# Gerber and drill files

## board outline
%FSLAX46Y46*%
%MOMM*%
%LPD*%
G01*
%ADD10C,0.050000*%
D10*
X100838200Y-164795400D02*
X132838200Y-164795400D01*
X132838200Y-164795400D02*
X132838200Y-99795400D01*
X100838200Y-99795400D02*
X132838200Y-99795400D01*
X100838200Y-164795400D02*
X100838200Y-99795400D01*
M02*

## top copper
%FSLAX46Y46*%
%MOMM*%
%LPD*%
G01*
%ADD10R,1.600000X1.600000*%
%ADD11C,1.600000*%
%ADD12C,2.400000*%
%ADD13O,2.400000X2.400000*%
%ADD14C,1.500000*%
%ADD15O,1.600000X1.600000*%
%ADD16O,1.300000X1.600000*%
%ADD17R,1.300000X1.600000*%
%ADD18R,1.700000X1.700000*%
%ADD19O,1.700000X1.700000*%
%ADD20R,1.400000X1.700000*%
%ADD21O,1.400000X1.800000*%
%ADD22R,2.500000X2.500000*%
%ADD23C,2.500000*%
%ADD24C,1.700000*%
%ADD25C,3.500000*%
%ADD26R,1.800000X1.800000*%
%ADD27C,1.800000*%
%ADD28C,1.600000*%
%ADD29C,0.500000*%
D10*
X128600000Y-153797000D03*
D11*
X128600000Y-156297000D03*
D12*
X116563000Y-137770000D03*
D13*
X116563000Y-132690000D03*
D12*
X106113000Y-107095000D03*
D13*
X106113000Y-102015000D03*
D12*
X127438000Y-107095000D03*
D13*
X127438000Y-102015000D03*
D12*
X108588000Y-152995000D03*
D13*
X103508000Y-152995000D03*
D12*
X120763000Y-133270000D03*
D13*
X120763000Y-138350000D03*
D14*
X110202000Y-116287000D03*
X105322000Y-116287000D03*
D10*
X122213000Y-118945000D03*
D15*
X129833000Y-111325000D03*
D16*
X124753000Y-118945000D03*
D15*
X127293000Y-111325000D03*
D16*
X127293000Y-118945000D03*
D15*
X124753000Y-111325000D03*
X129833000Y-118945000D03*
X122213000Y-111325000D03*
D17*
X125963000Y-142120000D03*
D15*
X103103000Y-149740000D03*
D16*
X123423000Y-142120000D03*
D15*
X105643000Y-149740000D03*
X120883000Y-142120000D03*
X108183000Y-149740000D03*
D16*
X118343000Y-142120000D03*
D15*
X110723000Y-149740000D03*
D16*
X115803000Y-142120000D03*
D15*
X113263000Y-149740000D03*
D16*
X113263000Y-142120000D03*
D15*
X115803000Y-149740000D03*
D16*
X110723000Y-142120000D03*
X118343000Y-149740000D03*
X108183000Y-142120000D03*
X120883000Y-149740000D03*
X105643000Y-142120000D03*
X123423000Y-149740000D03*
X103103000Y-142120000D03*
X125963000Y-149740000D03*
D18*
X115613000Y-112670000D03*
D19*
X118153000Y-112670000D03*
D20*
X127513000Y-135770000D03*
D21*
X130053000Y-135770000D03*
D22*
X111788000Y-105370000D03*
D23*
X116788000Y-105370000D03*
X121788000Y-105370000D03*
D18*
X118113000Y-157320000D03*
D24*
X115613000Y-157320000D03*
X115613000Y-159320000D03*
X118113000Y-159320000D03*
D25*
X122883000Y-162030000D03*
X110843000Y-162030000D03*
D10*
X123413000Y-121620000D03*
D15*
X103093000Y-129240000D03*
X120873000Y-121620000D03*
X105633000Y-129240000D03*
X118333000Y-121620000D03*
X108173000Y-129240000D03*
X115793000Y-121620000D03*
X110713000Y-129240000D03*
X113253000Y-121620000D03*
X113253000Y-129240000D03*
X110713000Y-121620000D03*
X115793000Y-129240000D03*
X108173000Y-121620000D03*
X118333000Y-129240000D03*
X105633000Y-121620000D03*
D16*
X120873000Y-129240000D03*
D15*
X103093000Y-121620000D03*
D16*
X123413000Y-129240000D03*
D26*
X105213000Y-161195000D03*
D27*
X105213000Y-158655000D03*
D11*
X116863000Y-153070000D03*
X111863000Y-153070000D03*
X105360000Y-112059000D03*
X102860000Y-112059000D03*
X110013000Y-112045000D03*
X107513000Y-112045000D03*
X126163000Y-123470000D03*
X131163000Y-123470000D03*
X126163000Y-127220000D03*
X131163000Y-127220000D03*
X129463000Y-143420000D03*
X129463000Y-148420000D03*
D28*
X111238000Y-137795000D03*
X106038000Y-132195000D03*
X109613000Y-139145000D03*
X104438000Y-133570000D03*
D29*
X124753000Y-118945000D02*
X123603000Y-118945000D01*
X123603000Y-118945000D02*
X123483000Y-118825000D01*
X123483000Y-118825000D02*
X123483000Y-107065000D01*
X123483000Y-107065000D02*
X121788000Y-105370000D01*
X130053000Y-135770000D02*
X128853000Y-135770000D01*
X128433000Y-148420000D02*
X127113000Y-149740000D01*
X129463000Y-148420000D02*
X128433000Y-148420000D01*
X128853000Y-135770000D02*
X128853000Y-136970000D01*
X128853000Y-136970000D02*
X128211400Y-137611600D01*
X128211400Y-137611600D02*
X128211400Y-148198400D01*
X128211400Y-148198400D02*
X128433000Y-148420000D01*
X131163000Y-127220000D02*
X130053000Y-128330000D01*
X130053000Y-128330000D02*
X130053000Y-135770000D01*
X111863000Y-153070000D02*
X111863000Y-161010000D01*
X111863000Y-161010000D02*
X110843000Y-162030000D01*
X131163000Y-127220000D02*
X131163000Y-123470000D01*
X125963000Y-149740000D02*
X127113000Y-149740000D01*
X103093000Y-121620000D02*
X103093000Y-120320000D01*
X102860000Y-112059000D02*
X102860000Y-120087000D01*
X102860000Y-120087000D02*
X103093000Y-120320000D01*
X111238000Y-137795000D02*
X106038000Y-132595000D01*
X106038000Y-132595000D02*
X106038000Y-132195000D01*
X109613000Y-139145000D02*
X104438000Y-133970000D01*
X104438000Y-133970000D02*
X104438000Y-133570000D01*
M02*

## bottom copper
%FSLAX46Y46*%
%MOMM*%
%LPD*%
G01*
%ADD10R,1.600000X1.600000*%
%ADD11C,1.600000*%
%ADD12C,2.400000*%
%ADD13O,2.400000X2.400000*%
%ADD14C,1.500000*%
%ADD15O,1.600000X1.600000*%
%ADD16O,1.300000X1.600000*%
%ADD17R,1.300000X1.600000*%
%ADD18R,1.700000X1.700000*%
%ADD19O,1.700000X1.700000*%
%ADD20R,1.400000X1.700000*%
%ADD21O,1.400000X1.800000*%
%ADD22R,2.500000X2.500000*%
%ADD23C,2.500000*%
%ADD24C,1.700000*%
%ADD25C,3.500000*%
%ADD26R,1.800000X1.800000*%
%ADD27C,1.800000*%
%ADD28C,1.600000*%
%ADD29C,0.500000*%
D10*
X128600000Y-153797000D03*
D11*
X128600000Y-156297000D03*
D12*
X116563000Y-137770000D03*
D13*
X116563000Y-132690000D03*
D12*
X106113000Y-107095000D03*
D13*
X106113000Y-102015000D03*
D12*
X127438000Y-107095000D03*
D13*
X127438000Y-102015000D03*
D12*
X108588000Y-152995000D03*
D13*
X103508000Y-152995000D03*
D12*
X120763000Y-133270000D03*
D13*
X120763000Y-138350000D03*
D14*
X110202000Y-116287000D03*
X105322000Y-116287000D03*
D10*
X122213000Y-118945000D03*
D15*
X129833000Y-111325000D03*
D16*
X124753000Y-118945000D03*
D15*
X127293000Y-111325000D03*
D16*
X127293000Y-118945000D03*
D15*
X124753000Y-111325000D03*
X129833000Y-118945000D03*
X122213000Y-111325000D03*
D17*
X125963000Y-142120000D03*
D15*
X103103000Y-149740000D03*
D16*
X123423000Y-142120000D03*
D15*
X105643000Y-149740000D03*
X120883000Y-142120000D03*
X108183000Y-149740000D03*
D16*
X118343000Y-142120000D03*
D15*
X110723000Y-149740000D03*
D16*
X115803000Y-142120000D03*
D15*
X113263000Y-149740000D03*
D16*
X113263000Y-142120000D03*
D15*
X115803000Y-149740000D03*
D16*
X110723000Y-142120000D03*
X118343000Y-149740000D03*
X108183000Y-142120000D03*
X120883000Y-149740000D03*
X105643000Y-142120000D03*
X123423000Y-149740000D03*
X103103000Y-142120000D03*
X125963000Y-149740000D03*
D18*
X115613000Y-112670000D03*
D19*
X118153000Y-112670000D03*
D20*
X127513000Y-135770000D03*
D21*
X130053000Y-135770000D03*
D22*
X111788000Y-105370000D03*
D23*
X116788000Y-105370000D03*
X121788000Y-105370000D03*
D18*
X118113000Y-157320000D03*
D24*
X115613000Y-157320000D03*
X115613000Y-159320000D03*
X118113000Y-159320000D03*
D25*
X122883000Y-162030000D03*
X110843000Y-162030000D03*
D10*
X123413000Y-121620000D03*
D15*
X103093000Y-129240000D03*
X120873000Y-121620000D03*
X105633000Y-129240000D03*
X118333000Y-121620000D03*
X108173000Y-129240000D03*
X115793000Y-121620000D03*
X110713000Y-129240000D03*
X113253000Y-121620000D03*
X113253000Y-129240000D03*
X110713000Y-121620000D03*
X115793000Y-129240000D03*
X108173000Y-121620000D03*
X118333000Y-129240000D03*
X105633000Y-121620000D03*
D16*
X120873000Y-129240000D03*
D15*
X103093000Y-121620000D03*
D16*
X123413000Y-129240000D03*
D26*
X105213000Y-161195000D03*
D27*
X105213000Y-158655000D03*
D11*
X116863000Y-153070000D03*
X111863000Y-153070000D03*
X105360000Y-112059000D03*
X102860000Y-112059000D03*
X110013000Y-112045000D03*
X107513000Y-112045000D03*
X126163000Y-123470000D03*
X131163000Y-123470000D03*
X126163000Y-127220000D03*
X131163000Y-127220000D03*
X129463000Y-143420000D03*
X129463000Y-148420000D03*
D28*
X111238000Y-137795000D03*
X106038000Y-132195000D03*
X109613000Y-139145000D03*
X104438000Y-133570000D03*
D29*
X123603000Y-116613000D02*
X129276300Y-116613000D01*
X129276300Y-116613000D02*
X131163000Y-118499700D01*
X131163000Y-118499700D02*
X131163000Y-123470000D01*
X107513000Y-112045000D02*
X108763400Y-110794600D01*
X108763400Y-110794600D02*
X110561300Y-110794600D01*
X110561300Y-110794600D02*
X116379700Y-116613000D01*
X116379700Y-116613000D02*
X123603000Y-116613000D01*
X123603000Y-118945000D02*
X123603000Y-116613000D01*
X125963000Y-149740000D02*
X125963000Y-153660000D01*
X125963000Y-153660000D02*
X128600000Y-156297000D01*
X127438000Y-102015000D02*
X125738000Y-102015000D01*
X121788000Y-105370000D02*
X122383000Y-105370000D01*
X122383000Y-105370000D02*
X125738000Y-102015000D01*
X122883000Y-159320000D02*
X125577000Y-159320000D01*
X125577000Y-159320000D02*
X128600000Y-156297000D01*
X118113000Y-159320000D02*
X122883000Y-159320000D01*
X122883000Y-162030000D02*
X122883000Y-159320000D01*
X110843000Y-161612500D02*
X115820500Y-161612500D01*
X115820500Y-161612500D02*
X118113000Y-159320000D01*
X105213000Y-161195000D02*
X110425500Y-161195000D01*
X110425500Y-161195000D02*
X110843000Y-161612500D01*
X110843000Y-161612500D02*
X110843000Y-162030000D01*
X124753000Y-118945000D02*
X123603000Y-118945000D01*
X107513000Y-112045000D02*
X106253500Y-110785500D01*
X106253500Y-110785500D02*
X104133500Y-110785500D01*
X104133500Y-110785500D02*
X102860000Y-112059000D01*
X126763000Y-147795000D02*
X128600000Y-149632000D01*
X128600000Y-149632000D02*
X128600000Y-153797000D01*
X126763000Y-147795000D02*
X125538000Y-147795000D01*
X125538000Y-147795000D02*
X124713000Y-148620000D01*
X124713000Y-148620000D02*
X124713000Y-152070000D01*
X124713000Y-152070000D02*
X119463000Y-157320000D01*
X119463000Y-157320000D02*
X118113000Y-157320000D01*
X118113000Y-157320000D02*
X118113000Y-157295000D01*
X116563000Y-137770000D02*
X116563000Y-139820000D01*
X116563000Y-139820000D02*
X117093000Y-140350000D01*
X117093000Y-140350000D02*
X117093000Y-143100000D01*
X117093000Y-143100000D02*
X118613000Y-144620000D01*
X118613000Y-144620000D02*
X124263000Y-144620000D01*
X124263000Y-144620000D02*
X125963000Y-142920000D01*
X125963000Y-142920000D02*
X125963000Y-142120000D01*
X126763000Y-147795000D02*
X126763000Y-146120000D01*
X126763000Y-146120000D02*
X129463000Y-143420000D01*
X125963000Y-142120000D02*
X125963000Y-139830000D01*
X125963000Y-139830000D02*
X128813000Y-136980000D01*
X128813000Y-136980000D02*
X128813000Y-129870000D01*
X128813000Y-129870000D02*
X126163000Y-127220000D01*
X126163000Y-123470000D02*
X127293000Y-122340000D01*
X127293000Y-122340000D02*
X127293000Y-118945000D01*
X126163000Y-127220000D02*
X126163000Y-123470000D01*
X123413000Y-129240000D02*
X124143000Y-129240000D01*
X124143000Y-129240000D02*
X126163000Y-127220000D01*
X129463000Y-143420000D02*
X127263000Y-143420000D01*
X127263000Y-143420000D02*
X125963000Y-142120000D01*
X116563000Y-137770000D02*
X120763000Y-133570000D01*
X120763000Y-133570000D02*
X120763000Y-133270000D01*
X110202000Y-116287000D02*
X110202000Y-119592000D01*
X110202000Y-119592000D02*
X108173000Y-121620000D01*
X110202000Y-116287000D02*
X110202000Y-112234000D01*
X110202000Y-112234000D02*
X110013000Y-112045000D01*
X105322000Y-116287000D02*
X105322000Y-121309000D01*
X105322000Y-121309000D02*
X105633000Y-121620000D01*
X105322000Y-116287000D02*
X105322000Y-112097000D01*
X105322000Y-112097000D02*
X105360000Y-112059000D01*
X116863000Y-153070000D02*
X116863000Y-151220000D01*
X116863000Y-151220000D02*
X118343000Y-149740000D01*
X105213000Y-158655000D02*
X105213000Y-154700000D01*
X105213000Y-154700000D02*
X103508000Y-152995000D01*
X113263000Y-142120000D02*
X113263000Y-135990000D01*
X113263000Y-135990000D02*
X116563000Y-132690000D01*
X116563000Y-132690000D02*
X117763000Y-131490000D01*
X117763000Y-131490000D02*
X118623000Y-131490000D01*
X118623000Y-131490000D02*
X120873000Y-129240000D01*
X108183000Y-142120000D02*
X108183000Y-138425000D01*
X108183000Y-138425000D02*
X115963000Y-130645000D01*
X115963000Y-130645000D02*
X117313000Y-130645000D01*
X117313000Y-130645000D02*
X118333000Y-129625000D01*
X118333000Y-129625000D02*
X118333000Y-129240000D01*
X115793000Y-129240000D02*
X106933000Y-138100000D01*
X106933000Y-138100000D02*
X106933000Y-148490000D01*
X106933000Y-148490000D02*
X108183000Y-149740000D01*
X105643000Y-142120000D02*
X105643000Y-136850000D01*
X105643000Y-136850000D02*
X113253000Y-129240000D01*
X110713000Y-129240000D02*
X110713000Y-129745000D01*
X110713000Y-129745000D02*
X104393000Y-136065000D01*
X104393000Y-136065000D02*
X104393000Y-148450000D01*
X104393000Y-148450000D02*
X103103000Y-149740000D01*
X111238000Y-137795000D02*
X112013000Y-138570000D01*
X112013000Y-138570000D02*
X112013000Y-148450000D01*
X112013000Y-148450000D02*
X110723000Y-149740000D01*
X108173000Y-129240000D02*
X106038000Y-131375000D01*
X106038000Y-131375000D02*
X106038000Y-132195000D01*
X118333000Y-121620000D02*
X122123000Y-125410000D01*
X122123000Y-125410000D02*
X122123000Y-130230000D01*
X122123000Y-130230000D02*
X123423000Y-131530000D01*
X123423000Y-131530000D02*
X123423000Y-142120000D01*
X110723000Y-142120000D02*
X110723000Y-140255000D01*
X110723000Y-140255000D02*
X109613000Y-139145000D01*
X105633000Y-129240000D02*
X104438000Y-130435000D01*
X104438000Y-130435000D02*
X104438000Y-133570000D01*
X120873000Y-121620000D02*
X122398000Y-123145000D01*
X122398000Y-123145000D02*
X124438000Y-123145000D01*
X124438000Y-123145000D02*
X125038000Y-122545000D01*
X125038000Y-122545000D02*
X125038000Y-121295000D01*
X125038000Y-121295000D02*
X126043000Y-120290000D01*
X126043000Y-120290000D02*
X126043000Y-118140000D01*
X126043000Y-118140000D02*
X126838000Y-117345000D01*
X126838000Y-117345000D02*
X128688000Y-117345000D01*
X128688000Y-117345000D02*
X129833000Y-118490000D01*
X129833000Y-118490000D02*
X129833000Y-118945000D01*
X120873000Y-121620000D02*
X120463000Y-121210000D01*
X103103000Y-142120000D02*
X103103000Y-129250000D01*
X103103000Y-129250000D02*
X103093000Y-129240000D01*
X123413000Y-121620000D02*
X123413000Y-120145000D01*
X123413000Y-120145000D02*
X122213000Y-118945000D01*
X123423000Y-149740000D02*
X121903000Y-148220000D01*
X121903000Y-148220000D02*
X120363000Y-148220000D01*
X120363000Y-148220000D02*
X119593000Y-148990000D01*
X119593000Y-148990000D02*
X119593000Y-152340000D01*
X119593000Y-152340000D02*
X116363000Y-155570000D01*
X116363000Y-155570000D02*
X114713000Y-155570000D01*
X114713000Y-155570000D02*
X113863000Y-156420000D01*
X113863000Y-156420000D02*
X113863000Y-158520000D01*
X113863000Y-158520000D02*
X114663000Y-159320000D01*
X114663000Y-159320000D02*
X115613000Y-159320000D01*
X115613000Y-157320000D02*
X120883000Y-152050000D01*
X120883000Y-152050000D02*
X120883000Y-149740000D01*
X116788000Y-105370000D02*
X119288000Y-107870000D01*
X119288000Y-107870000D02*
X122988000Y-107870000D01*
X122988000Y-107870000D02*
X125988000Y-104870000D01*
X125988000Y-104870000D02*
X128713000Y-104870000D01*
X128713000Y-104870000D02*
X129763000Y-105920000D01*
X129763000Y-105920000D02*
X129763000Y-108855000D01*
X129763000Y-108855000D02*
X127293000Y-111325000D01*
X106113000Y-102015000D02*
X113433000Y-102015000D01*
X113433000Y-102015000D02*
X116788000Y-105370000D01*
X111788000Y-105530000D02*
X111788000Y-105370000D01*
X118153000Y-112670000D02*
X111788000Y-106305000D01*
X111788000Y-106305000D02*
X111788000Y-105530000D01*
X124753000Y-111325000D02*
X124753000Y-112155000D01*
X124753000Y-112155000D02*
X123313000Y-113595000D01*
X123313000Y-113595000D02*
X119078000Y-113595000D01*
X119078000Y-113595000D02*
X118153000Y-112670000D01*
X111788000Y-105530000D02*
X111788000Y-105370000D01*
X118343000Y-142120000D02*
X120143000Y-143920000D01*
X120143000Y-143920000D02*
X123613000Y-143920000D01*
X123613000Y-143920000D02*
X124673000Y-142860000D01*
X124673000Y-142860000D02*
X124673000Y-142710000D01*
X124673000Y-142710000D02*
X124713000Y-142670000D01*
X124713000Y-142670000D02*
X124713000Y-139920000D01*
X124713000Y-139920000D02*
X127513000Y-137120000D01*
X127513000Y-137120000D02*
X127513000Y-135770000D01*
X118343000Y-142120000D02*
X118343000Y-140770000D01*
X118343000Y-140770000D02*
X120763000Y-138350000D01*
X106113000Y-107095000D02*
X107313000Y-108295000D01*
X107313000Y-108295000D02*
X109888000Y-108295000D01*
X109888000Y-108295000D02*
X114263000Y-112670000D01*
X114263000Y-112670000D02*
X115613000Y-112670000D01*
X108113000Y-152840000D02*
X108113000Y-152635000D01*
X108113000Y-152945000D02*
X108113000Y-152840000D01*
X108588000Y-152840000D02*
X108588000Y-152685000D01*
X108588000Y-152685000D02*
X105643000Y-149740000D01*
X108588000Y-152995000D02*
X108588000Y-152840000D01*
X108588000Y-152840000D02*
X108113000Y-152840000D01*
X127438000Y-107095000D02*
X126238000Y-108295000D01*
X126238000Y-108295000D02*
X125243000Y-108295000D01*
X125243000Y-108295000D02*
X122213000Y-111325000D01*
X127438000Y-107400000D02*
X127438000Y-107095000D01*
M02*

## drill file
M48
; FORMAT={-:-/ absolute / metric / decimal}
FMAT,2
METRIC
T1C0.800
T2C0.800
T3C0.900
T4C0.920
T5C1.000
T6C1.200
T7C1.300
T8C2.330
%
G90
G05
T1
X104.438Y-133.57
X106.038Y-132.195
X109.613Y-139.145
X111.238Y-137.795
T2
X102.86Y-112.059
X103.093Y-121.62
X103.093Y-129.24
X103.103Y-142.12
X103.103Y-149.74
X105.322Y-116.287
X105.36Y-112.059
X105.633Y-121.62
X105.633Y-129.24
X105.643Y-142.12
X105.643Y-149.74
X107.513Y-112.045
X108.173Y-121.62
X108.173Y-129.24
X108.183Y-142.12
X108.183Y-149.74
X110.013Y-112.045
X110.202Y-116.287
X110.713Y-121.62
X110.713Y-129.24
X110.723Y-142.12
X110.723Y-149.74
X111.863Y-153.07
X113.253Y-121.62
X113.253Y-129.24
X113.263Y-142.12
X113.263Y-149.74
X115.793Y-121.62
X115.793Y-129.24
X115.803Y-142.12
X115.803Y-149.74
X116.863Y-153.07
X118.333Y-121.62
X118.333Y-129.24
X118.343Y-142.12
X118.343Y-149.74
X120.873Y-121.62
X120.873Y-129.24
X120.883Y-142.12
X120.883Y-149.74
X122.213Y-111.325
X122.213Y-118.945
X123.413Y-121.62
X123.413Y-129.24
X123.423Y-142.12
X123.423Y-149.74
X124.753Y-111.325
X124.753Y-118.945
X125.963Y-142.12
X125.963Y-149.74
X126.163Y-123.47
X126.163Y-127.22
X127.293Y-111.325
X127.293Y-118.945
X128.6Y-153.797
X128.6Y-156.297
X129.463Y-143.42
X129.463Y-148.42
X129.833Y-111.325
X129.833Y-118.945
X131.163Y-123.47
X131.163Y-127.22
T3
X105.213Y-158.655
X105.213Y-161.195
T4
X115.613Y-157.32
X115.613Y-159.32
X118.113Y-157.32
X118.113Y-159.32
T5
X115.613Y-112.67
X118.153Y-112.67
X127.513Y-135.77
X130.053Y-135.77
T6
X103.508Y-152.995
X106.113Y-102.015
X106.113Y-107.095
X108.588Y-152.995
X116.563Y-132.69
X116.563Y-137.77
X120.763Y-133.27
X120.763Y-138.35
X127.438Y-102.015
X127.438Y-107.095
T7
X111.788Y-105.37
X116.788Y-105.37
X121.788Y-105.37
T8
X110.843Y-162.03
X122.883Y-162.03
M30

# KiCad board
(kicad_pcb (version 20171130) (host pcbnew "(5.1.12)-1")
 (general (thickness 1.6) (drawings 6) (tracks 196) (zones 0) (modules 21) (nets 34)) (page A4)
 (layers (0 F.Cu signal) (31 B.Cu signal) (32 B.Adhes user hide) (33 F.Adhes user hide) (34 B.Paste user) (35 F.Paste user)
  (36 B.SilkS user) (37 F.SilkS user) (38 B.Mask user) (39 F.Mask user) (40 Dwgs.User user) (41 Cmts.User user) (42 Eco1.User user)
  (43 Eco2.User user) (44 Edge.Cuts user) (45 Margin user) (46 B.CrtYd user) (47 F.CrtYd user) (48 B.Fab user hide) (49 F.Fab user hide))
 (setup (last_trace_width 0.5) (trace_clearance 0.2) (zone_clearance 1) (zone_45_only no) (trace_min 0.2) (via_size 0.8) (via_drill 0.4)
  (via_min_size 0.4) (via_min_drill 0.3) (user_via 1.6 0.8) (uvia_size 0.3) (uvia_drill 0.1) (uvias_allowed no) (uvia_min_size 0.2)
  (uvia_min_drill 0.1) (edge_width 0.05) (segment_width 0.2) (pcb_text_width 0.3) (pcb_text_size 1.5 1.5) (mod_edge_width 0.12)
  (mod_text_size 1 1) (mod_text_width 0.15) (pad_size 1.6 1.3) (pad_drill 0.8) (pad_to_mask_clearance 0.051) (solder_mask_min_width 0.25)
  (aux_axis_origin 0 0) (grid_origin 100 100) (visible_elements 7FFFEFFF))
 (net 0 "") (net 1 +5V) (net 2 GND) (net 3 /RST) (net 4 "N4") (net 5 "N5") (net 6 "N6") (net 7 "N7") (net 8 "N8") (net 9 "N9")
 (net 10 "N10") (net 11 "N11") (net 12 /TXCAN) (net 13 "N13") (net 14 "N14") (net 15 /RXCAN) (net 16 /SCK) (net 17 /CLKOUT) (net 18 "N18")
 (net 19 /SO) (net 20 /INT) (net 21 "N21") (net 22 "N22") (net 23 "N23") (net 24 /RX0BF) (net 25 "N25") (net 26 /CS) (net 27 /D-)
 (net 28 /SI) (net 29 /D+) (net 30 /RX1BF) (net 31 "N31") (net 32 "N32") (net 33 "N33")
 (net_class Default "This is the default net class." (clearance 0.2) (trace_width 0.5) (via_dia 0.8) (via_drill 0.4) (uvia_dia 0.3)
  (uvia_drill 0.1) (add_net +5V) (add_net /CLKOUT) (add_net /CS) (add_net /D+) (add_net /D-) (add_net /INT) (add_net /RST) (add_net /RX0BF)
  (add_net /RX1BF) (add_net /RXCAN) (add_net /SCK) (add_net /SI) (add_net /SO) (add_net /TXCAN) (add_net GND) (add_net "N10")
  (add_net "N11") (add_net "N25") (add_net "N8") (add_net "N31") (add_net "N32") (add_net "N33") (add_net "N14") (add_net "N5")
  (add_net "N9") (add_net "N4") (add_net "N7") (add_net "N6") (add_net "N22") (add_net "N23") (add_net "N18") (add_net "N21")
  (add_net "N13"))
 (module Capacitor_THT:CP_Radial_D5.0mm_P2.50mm (layer F.Cu) (at 128.6 153.797 270)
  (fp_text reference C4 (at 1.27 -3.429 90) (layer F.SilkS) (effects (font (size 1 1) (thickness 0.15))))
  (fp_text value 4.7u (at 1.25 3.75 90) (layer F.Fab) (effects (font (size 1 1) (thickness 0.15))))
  (pad 1 thru_hole rect (at 0 0 270) (size 1.6 1.6) (drill 0.8) (layers *.Cu *.Mask) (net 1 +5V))
  (pad 2 thru_hole circle (at 2.5 0 270) (size 1.6 1.6) (drill 0.8) (layers *.Cu *.Mask) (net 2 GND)))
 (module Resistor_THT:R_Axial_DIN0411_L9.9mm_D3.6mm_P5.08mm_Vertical (layer F.Cu) (at 116.563 137.77 90)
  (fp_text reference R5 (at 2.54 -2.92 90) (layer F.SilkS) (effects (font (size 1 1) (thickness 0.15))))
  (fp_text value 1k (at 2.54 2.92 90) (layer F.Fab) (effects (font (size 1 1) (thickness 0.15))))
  (pad 1 thru_hole circle (at 0 0 90) (size 2.4 2.4) (drill 1.2) (layers *.Cu *.Mask) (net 1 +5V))
  (pad 2 thru_hole oval (at 5.08 0 90) (size 2.4 2.4) (drill 1.2) (layers *.Cu *.Mask) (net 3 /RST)))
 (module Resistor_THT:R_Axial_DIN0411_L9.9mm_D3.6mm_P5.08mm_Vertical (layer F.Cu) (at 106.113 107.095 90)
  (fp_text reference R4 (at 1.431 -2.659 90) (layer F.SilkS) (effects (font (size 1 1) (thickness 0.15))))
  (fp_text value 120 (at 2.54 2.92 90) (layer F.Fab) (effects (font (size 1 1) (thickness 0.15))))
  (pad 1 thru_hole circle (at 0 0 90) (size 2.4 2.4) (drill 1.2) (layers *.Cu *.Mask) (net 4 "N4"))
  (pad 2 thru_hole oval (at 5.08 0 90) (size 2.4 2.4) (drill 1.2) (layers *.Cu *.Mask) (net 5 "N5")))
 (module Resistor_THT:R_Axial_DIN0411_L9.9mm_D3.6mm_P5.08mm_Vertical (layer F.Cu) (at 127.438 107.095 90)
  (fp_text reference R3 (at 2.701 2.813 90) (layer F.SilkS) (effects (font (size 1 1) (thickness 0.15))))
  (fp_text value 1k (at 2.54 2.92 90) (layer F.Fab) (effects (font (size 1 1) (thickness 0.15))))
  (pad 1 thru_hole circle (at 0 0 90) (size 2.4 2.4) (drill 1.2) (layers *.Cu *.Mask) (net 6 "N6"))
  (pad 2 thru_hole oval (at 5.08 0 90) (size 2.4 2.4) (drill 1.2) (layers *.Cu *.Mask) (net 2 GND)))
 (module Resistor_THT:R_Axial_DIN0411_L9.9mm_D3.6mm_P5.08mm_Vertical (layer F.Cu) (at 108.588 152.995 180)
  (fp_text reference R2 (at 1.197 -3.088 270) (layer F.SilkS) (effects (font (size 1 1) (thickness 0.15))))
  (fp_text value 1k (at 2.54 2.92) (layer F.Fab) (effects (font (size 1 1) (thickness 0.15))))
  (pad 1 thru_hole circle (at 0 0 180) (size 2.4 2.4) (drill 1.2) (layers *.Cu *.Mask) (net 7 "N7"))
  (pad 2 thru_hole oval (at 5.08 0 180) (size 2.4 2.4) (drill 1.2) (layers *.Cu *.Mask) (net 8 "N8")))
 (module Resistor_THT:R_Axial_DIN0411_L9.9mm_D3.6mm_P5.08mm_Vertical (layer F.Cu) (at 120.763 133.27 270)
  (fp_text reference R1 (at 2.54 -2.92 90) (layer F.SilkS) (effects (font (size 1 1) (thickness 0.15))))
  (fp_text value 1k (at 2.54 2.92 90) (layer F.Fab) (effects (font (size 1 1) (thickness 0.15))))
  (pad 1 thru_hole circle (at 0 0 270) (size 2.4 2.4) (drill 1.2) (layers *.Cu *.Mask) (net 1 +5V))
  (pad 2 thru_hole oval (at 5.08 0 270) (size 2.4 2.4) (drill 1.2) (layers *.Cu *.Mask) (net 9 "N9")))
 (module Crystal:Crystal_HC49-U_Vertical (layer F.Cu) (at 110.202 116.287 180)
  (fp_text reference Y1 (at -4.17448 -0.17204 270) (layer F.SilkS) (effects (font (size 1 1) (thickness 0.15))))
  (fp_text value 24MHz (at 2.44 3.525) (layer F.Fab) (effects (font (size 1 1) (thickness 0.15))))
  (pad 1 thru_hole circle (at 0 0 180) (size 1.5 1.5) (drill 0.8) (layers *.Cu *.Mask) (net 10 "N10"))
  (pad 2 thru_hole circle (at 4.88 0 180) (size 1.5 1.5) (drill 0.8) (layers *.Cu *.Mask) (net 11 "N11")))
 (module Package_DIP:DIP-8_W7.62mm (layer F.Cu) (at 122.213 118.945 90)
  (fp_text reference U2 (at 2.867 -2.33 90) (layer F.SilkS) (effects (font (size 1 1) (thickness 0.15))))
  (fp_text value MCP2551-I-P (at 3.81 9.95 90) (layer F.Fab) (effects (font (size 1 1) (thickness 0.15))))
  (pad 1 thru_hole rect (at 0 0 90) (size 1.6 1.6) (drill 0.8) (layers *.Cu *.Mask) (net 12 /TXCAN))
  (pad 5 thru_hole oval (at 7.62 7.62 90) (size 1.6 1.6) (drill 0.8) (layers *.Cu *.Mask) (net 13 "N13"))
  (pad 2 thru_hole oval (at 0 2.54 90) (size 1.6 1.3) (drill 0.8) (layers *.Cu *.Mask) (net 2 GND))
  (pad 6 thru_hole oval (at 7.62 5.08 90) (size 1.6 1.6) (drill 0.8) (layers *.Cu *.Mask) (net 5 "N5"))
  (pad 3 thru_hole oval (at 0 5.08 90) (size 1.6 1.3) (drill 0.8) (layers *.Cu *.Mask) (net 1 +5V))
  (pad 7 thru_hole oval (at 7.62 2.54 90) (size 1.6 1.6) (drill 0.8) (layers *.Cu *.Mask) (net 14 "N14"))
  (pad 4 thru_hole oval (at 0 7.62 90) (size 1.6 1.6) (drill 0.8) (layers *.Cu *.Mask) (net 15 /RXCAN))
  (pad 8 thru_hole oval (at 7.62 0 90) (size 1.6 1.6) (drill 0.8) (layers *.Cu *.Mask) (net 6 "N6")))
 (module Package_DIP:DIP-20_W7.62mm (layer F.Cu) (at 125.963 142.12 270)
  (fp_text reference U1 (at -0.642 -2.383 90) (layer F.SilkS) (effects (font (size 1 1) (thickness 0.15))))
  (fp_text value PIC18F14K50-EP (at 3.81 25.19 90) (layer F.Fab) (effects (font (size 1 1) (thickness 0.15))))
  (pad 1 thru_hole rect (at 0 0 270) (size 1.6 1.3) (drill 0.8) (layers *.Cu *.Mask) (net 1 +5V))
  (pad 11 thru_hole oval (at 7.62 22.86 270) (size 1.6 1.6) (drill 0.8) (layers *.Cu *.Mask) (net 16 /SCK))
  (pad 2 thru_hole oval (at 0 2.54 270) (size 1.6 1.3) (drill 0.8) (layers *.Cu *.Mask) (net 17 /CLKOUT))
  (pad 12 thru_hole oval (at 7.62 20.32 270) (size 1.6 1.6) (drill 0.8) (layers *.Cu *.Mask) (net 7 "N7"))
  (pad 3 thru_hole oval (at 0 5.08 270) (size 1.6 1.6) (drill 0.8) (layers *.Cu *.Mask) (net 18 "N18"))
  (pad 13 thru_hole oval (at 7.62 17.78 270) (size 1.6 1.6) (drill 0.8) (layers *.Cu *.Mask) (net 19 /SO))
  (pad 4 thru_hole oval (at 0 7.62 270) (size 1.6 1.3) (drill 0.8) (layers *.Cu *.Mask) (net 9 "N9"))
  (pad 14 thru_hole oval (at 7.62 15.24 270) (size 1.6 1.6) (drill 0.8) (layers *.Cu *.Mask) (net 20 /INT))
  (pad 5 thru_hole oval (at 0 10.16 270) (size 1.6 1.3) (drill 0.8) (layers *.Cu *.Mask) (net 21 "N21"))
  (pad 15 thru_hole oval (at 7.62 12.7 270) (size 1.6 1.6) (drill 0.8) (layers *.Cu *.Mask) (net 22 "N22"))
  (pad 6 thru_hole oval (at 0 12.7 270) (size 1.6 1.3) (drill 0.8) (layers *.Cu *.Mask) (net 3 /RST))
  (pad 16 thru_hole oval (at 7.62 10.16 270) (size 1.6 1.6) (drill 0.8) (layers *.Cu *.Mask) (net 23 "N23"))
  (pad 7 thru_hole oval (at 0 15.24 270) (size 1.6 1.3) (drill 0.8) (layers *.Cu *.Mask) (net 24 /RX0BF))
  (pad 17 thru_hole oval (at 7.62 7.62 270) (size 1.6 1.3) (drill 0.8) (layers *.Cu *.Mask) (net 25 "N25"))
  (pad 8 thru_hole oval (at 0 17.78 270) (size 1.6 1.3) (drill 0.8) (layers *.Cu *.Mask) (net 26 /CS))
  (pad 18 thru_hole oval (at 7.62 5.08 270) (size 1.6 1.3) (drill 0.8) (layers *.Cu *.Mask) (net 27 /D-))
  (pad 9 thru_hole oval (at 0 20.32 270) (size 1.6 1.3) (drill 0.8) (layers *.Cu *.Mask) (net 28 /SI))
  (pad 19 thru_hole oval (at 7.62 2.54 270) (size 1.6 1.3) (drill 0.8) (layers *.Cu *.Mask) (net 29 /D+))
  (pad 10 thru_hole oval (at 0 22.86 270) (size 1.6 1.3) (drill 0.8) (layers *.Cu *.Mask) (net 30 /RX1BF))
  (pad 20 thru_hole oval (at 7.62 0 270) (size 1.6 1.3) (drill 0.8) (layers *.Cu *.Mask) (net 2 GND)))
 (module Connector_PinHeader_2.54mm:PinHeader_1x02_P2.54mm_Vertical (layer F.Cu) (at 115.613 112.67 90)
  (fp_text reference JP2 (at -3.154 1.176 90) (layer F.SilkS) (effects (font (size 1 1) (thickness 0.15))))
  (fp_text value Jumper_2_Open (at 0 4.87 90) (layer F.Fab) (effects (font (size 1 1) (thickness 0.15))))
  (pad 1 thru_hole rect (at 0 0 90) (size 1.7 1.7) (drill 1) (layers *.Cu *.Mask) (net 4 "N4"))
  (pad 2 thru_hole oval (at 0 2.54 90) (size 1.7 1.7) (drill 1) (layers *.Cu *.Mask) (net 14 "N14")))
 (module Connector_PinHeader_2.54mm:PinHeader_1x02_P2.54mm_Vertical (layer F.Cu) (at 127.513 135.77 90)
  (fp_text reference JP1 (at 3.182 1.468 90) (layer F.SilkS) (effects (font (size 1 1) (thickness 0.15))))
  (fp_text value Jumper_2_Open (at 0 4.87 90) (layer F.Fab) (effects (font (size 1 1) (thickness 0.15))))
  (pad 1 thru_hole rect (at 0 0 90) (size 1.7 1.4) (drill 1) (layers *.Cu *.Mask) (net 9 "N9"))
  (pad 2 thru_hole oval (at 0 2.54 90) (size 1.8 1.4) (drill 1) (layers *.Cu *.Mask) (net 2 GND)))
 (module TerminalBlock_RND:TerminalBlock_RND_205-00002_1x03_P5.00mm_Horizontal (layer F.Cu) (at 111.788 105.37)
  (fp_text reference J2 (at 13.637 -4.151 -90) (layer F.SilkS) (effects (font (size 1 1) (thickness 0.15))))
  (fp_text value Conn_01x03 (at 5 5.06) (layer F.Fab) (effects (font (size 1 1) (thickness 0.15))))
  (pad 1 thru_hole rect (at 0 0) (size 2.5 2.5) (drill 1.3) (layers *.Cu *.Mask) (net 14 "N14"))
  (pad 2 thru_hole circle (at 5 0) (size 2.5 2.5) (drill 1.3) (layers *.Cu *.Mask) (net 5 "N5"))
  (pad 3 thru_hole circle (at 10 0) (size 2.5 2.5) (drill 1.3) (layers *.Cu *.Mask) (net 2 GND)))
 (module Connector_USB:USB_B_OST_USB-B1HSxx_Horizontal (layer F.Cu) (at 118.113 157.32 270)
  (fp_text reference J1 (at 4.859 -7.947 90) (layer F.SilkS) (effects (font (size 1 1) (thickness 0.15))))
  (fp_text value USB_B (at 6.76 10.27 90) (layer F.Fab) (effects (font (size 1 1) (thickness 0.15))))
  (pad 1 thru_hole rect (at 0 0 270) (size 1.7 1.7) (drill 0.92) (layers *.Cu *.Mask) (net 1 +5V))
  (pad 2 thru_hole circle (at 0 2.5 270) (size 1.7 1.7) (drill 0.92) (layers *.Cu *.Mask) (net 27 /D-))
  (pad 3 thru_hole circle (at 2 2.5 270) (size 1.7 1.7) (drill 0.92) (layers *.Cu *.Mask) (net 29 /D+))
  (pad 4 thru_hole circle (at 2 0 270) (size 1.7 1.7) (drill 0.92) (layers *.Cu *.Mask) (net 2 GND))
  (pad 5 thru_hole circle (at 4.71 -4.77 270) (size 3.5 3.5) (drill 2.33) (layers *.Cu *.Mask) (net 2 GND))
  (pad 5 thru_hole circle (at 4.71 7.27 270) (size 3.5 3.5) (drill 2.33) (layers *.Cu *.Mask) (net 2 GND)))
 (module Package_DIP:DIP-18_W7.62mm (layer F.Cu) (at 123.413 121.62 270)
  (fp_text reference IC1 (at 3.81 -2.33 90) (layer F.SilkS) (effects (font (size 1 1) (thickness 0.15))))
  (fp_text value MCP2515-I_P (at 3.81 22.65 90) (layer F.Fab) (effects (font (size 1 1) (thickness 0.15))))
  (pad 1 thru_hole rect (at 0 0 270) (size 1.6 1.6) (drill 0.8) (layers *.Cu *.Mask) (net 12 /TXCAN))
  (pad 10 thru_hole oval (at 7.62 20.32 270) (size 1.6 1.6) (drill 0.8) (layers *.Cu *.Mask) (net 30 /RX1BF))
  (pad 2 thru_hole oval (at 0 2.54 270) (size 1.6 1.6) (drill 0.8) (layers *.Cu *.Mask) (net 15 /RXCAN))
  (pad 11 thru_hole oval (at 7.62 17.78 270) (size 1.6 1.6) (drill 0.8) (layers *.Cu *.Mask) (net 24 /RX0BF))
  (pad 3 thru_hole oval (at 0 5.08 270) (size 1.6 1.6) (drill 0.8) (layers *.Cu *.Mask) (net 17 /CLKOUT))
  (pad 12 thru_hole oval (at 7.62 15.24 270) (size 1.6 1.6) (drill 0.8) (layers *.Cu *.Mask) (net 20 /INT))
  (pad 4 thru_hole oval (at 0 7.62 270) (size 1.6 1.6) (drill 0.8) (layers *.Cu *.Mask) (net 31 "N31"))
  (pad 13 thru_hole oval (at 7.62 12.7 270) (size 1.6 1.6) (drill 0.8) (layers *.Cu *.Mask) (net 16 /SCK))
  (pad 5 thru_hole oval (at 0 10.16 270) (size 1.6 1.6) (drill 0.8) (layers *.Cu *.Mask) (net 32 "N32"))
  (pad 14 thru_hole oval (at 7.62 10.16 270) (size 1.6 1.6) (drill 0.8) (layers *.Cu *.Mask) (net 28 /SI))
  (pad 6 thru_hole oval (at 0 12.7 270) (size 1.6 1.6) (drill 0.8) (layers *.Cu *.Mask) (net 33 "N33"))
  (pad 15 thru_hole oval (at 7.62 7.62 270) (size 1.6 1.6) (drill 0.8) (layers *.Cu *.Mask) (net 19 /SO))
  (pad 7 thru_hole oval (at 0 15.24 270) (size 1.6 1.6) (drill 0.8) (layers *.Cu *.Mask) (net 10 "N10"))
  (pad 16 thru_hole oval (at 7.62 5.08 270) (size 1.6 1.6) (drill 0.8) (layers *.Cu *.Mask) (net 26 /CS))
  (pad 8 thru_hole oval (at 0 17.78 270) (size 1.6 1.6) (drill 0.8) (layers *.Cu *.Mask) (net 11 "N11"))
  (pad 17 thru_hole oval (at 7.62 2.54 270) (size 1.6 1.3) (drill 0.8) (layers *.Cu *.Mask) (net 3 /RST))
  (pad 9 thru_hole oval (at 0 20.32 270) (size 1.6 1.6) (drill 0.8) (layers *.Cu *.Mask) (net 2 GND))
  (pad 18 thru_hole oval (at 7.62 0 270) (size 1.6 1.3) (drill 0.8) (layers *.Cu *.Mask) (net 1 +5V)))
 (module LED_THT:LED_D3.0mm (layer F.Cu) (at 105.213 161.195 90)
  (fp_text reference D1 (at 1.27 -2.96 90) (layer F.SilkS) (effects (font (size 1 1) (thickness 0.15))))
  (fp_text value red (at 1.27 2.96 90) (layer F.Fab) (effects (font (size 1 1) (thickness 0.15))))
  (pad 1 thru_hole rect (at 0 0 90) (size 1.8 1.8) (drill 0.9) (layers *.Cu *.Mask) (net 2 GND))
  (pad 2 thru_hole circle (at 2.54 0 90) (size 1.8 1.8) (drill 0.9) (layers *.Cu *.Mask) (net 8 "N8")))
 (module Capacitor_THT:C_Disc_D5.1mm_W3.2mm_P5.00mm (layer F.Cu) (at 116.863 153.07 180)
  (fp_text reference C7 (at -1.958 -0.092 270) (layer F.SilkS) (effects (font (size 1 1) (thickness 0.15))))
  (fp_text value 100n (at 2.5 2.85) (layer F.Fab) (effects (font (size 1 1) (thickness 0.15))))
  (pad 1 thru_hole circle (at 0 0 180) (size 1.6 1.6) (drill 0.8) (layers *.Cu *.Mask) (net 25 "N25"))
  (pad 2 thru_hole circle (at 5 0 180) (size 1.6 1.6) (drill 0.8) (layers *.Cu *.Mask) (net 2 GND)))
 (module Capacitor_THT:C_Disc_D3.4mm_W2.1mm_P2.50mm (layer F.Cu) (at 105.36 112.059 180)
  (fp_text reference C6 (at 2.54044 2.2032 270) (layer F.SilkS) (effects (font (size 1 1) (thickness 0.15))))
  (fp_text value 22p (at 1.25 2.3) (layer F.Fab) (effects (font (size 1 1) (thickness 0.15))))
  (pad 1 thru_hole circle (at 0 0 180) (size 1.6 1.6) (drill 0.8) (layers *.Cu *.Mask) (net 11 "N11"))
  (pad 2 thru_hole circle (at 2.5 0 180) (size 1.6 1.6) (drill 0.8) (layers *.Cu *.Mask) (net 2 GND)))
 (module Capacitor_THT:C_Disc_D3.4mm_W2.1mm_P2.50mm (layer F.Cu) (at 110.013 112.045 180)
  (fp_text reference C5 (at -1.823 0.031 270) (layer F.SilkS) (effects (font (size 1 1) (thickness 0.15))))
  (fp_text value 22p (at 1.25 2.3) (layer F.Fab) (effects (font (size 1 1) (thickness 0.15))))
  (pad 1 thru_hole circle (at 0 0 180) (size 1.6 1.6) (drill 0.8) (layers *.Cu *.Mask) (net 10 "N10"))
  (pad 2 thru_hole circle (at 2.5 0 180) (size 1.6 1.6) (drill 0.8) (layers *.Cu *.Mask) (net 2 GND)))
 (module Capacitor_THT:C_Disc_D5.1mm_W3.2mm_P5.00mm (layer F.Cu) (at 126.163 123.47)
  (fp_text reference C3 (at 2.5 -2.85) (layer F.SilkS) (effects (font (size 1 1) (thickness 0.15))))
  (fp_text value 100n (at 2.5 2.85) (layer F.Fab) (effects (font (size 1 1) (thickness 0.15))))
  (pad 1 thru_hole circle (at 0 0) (size 1.6 1.6) (drill 0.8) (layers *.Cu *.Mask) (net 1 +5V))
  (pad 2 thru_hole circle (at 5 0) (size 1.6 1.6) (drill 0.8) (layers *.Cu *.Mask) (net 2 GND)))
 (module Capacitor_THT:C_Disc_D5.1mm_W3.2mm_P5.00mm (layer F.Cu) (at 126.163 127.22)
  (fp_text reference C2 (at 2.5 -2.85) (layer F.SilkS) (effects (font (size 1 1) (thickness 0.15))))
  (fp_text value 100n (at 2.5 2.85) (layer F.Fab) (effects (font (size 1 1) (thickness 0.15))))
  (pad 1 thru_hole circle (at 0 0) (size 1.6 1.6) (drill 0.8) (layers *.Cu *.Mask) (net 1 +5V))
  (pad 2 thru_hole circle (at 5 0) (size 1.6 1.6) (drill 0.8) (layers *.Cu *.Mask) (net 2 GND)))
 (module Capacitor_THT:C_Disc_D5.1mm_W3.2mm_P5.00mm (layer F.Cu) (at 129.463 143.42 270)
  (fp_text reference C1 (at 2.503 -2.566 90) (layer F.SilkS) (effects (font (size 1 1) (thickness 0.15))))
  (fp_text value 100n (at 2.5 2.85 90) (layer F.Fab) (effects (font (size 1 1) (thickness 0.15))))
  (pad 1 thru_hole circle (at 0 0 270) (size 1.6 1.6) (drill 0.8) (layers *.Cu *.Mask) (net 1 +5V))
  (pad 2 thru_hole circle (at 5 0 270) (size 1.6 1.6) (drill 0.8) (layers *.Cu *.Mask) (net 2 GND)))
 (gr_line (start 100.8382 164.7954) (end 132.8382 164.7954) (layer Edge.Cuts) (width 0.05))
 (gr_line (start 132.8382 164.7954) (end 132.8382 99.7954) (layer Edge.Cuts) (width 0.05))
 (gr_line (start 100.8382 99.7954) (end 132.8382 99.7954) (layer Edge.Cuts) (width 0.05))
 (gr_line (start 100.8382 164.7954) (end 100.8382 99.7954) (layer Edge.Cuts) (width 0.05))
 (segment (start 123.603 116.613) (end 129.2763 116.613) (width 0.5) (layer B.Cu) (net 2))
 (segment (start 129.2763 116.613) (end 131.163 118.4997) (width 0.5) (layer B.Cu) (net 2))
 (segment (start 131.163 118.4997) (end 131.163 123.47) (width 0.5) (layer B.Cu) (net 2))
 (segment (start 107.513 112.045) (end 108.7634 110.7946) (width 0.5) (layer B.Cu) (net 2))
 (segment (start 108.7634 110.7946) (end 110.5613 110.7946) (width 0.5) (layer B.Cu) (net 2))
 (segment (start 110.5613 110.7946) (end 116.3797 116.613) (width 0.5) (layer B.Cu) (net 2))
 (segment (start 116.3797 116.613) (end 123.603 116.613) (width 0.5) (layer B.Cu) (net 2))
 (segment (start 123.603 118.945) (end 123.603 116.613) (width 0.5) (layer B.Cu) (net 2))
 (segment (start 124.753 118.945) (end 123.603 118.945) (width 0.5) (layer F.Cu) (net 2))
 (segment (start 123.603 118.945) (end 123.483 118.825) (width 0.5) (layer F.Cu) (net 2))
 (segment (start 123.483 118.825) (end 123.483 107.065) (width 0.5) (layer F.Cu) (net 2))
 (segment (start 123.483 107.065) (end 121.788 105.37) (width 0.5) (layer F.Cu) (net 2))
 (segment (start 125.963 149.74) (end 125.963 153.66) (width 0.5) (layer B.Cu) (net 2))
 (segment (start 125.963 153.66) (end 128.6 156.297) (width 0.5) (layer B.Cu) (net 2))
 (segment (start 130.053 135.77) (end 128.853 135.77) (width 0.5) (layer F.Cu) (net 2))
 (segment (start 128.433 148.42) (end 127.113 149.74) (width 0.5) (layer F.Cu) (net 2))
 (segment (start 129.463 148.42) (end 128.433 148.42) (width 0.5) (layer F.Cu) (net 2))
 (segment (start 128.853 135.77) (end 128.853 136.97) (width 0.5) (layer F.Cu) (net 2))
 (segment (start 128.853 136.97) (end 128.2114 137.6116) (width 0.5) (layer F.Cu) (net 2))
 (segment (start 128.2114 137.6116) (end 128.2114 148.1984) (width 0.5) (layer F.Cu) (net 2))
 (segment (start 128.2114 148.1984) (end 128.433 148.42) (width 0.5) (layer F.Cu) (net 2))
 (segment (start 131.163 127.22) (end 130.053 128.33) (width 0.5) (layer F.Cu) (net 2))
 (segment (start 130.053 128.33) (end 130.053 135.77) (width 0.5) (layer F.Cu) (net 2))
 (segment (start 127.438 102.015) (end 125.738 102.015) (width 0.5) (layer B.Cu) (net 2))
 (segment (start 121.788 105.37) (end 122.383 105.37) (width 0.5) (layer B.Cu) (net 2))
 (segment (start 122.383 105.37) (end 125.738 102.015) (width 0.5) (layer B.Cu) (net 2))
 (segment (start 122.883 159.32) (end 125.577 159.32) (width 0.5) (layer B.Cu) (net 2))
 (segment (start 125.577 159.32) (end 128.6 156.297) (width 0.5) (layer B.Cu) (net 2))
 (segment (start 118.113 159.32) (end 122.883 159.32) (width 0.5) (layer B.Cu) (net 2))
 (segment (start 122.883 162.03) (end 122.883 159.32) (width 0.5) (layer B.Cu) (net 2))
 (segment (start 110.843 161.6125) (end 115.8205 161.6125) (width 0.5) (layer B.Cu) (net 2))
 (segment (start 115.8205 161.6125) (end 118.113 159.32) (width 0.5) (layer B.Cu) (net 2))
 (segment (start 105.213 161.195) (end 110.4255 161.195) (width 0.5) (layer B.Cu) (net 2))
 (segment (start 110.4255 161.195) (end 110.843 161.6125) (width 0.5) (layer B.Cu) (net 2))
 (segment (start 110.843 161.6125) (end 110.843 162.03) (width 0.5) (layer B.Cu) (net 2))
 (segment (start 124.753 118.945) (end 123.603 118.945) (width 0.5) (layer B.Cu) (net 2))
 (segment (start 107.513 112.045) (end 106.2535 110.7855) (width 0.5) (layer B.Cu) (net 2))
 (segment (start 106.2535 110.7855) (end 104.1335 110.7855) (width 0.5) (layer B.Cu) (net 2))
 (segment (start 104.1335 110.7855) (end 102.86 112.059) (width 0.5) (layer B.Cu) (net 2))
 (segment (start 111.863 153.07) (end 111.863 161.01) (width 0.5) (layer F.Cu) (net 2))
 (segment (start 111.863 161.01) (end 110.843 162.03) (width 0.5) (layer F.Cu) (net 2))
 (segment (start 131.163 127.22) (end 131.163 123.47) (width 0.5) (layer F.Cu) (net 2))
 (segment (start 125.963 149.74) (end 127.113 149.74) (width 0.5) (layer F.Cu) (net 2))
 (segment (start 103.093 121.62) (end 103.093 120.32) (width 0.5) (layer F.Cu) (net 2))
 (segment (start 102.86 112.059) (end 102.86 120.087) (width 0.5) (layer F.Cu) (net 2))
 (segment (start 102.86 120.087) (end 103.093 120.32) (width 0.5) (layer F.Cu) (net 2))
 (segment (start 126.763 147.795) (end 128.6 149.632) (width 0.5) (layer B.Cu) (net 1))
 (segment (start 128.6 149.632) (end 128.6 153.797) (width 0.5) (layer B.Cu) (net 1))
 (segment (start 126.763 147.795) (end 125.538 147.795) (width 0.5) (layer B.Cu) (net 1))
 (segment (start 125.538 147.795) (end 124.713 148.62) (width 0.5) (layer B.Cu) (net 1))
 (segment (start 124.713 148.62) (end 124.713 152.07) (width 0.5) (layer B.Cu) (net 1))
 (segment (start 124.713 152.07) (end 119.463 157.32) (width 0.5) (layer B.Cu) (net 1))
 (segment (start 119.463 157.32) (end 118.113 157.32) (width 0.5) (layer B.Cu) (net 1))
 (segment (start 118.113 157.32) (end 118.113 157.295) (width 0.5) (layer B.Cu) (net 1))
 (segment (start 116.563 137.77) (end 116.563 139.82) (width 0.5) (layer B.Cu) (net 1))
 (segment (start 116.563 139.82) (end 117.093 140.35) (width 0.5) (layer B.Cu) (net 1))
 (segment (start 117.093 140.35) (end 117.093 143.1) (width 0.5) (layer B.Cu) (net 1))
 (segment (start 117.093 143.1) (end 118.613 144.62) (width 0.5) (layer B.Cu) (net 1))
 (segment (start 118.613 144.62) (end 124.263 144.62) (width 0.5) (layer B.Cu) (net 1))
 (segment (start 124.263 144.62) (end 125.963 142.92) (width 0.5) (layer B.Cu) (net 1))
 (segment (start 125.963 142.92) (end 125.963 142.12) (width 0.5) (layer B.Cu) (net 1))
 (segment (start 126.763 147.795) (end 126.763 146.12) (width 0.5) (layer B.Cu) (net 1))
 (segment (start 126.763 146.12) (end 129.463 143.42) (width 0.5) (layer B.Cu) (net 1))
 (segment (start 125.963 142.12) (end 125.963 139.83) (width 0.5) (layer B.Cu) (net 1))
 (segment (start 125.963 139.83) (end 128.813 136.98) (width 0.5) (layer B.Cu) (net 1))
 (segment (start 128.813 136.98) (end 128.813 129.87) (width 0.5) (layer B.Cu) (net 1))
 (segment (start 128.813 129.87) (end 126.163 127.22) (width 0.5) (layer B.Cu) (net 1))
 (segment (start 126.163 123.47) (end 127.293 122.34) (width 0.5) (layer B.Cu) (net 1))
 (segment (start 127.293 122.34) (end 127.293 118.945) (width 0.5) (layer B.Cu) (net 1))
 (segment (start 126.163 127.22) (end 126.163 123.47) (width 0.5) (layer B.Cu) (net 1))
 (segment (start 123.413 129.24) (end 124.143 129.24) (width 0.5) (layer B.Cu) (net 1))
 (segment (start 124.143 129.24) (end 126.163 127.22) (width 0.5) (layer B.Cu) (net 1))
 (segment (start 129.463 143.42) (end 127.263 143.42) (width 0.5) (layer B.Cu) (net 1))
 (segment (start 127.263 143.42) (end 125.963 142.12) (width 0.5) (layer B.Cu) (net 1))
 (segment (start 116.563 137.77) (end 120.763 133.57) (width 0.5) (layer B.Cu) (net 1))
 (segment (start 120.763 133.57) (end 120.763 133.27) (width 0.5) (layer B.Cu) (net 1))
 (segment (start 110.202 116.287) (end 110.202 119.592) (width 0.5) (layer B.Cu) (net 10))
 (segment (start 110.202 119.592) (end 108.173 121.62) (width 0.5) (layer B.Cu) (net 10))
 (segment (start 110.202 116.287) (end 110.202 112.234) (width 0.5) (layer B.Cu) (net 10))
 (segment (start 110.202 112.234) (end 110.013 112.045) (width 0.5) (layer B.Cu) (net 10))
 (segment (start 105.322 116.287) (end 105.322 121.309) (width 0.5) (layer B.Cu) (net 11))
 (segment (start 105.322 121.309) (end 105.633 121.62) (width 0.5) (layer B.Cu) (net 11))
 (segment (start 105.322 116.287) (end 105.322 112.097) (width 0.5) (layer B.Cu) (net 11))
 (segment (start 105.322 112.097) (end 105.36 112.059) (width 0.5) (layer B.Cu) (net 11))
 (segment (start 116.863 153.07) (end 116.863 151.22) (width 0.5) (layer B.Cu) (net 25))
 (segment (start 116.863 151.22) (end 118.343 149.74) (width 0.5) (layer B.Cu) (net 25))
 (segment (start 105.213 158.655) (end 105.213 154.7) (width 0.5) (layer B.Cu) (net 8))
 (segment (start 105.213 154.7) (end 103.508 152.995) (width 0.5) (layer B.Cu) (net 8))
 (segment (start 113.263 142.12) (end 113.263 135.99) (width 0.5) (layer B.Cu) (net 3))
 (segment (start 113.263 135.99) (end 116.563 132.69) (width 0.5) (layer B.Cu) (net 3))
 (segment (start 116.563 132.69) (end 117.763 131.49) (width 0.5) (layer B.Cu) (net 3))
 (segment (start 117.763 131.49) (end 118.623 131.49) (width 0.5) (layer B.Cu) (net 3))
 (segment (start 118.623 131.49) (end 120.873 129.24) (width 0.5) (layer B.Cu) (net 3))
 (segment (start 108.183 142.12) (end 108.183 138.425) (width 0.5) (layer B.Cu) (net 26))
 (segment (start 108.183 138.425) (end 115.963 130.645) (width 0.5) (layer B.Cu) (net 26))
 (segment (start 115.963 130.645) (end 117.313 130.645) (width 0.5) (layer B.Cu) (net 26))
 (segment (start 117.313 130.645) (end 118.333 129.625) (width 0.5) (layer B.Cu) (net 26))
 (segment (start 118.333 129.625) (end 118.333 129.24) (width 0.5) (layer B.Cu) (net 26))
 (segment (start 115.793 129.24) (end 106.933 138.1) (width 0.5) (layer B.Cu) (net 19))
 (segment (start 106.933 138.1) (end 106.933 148.49) (width 0.5) (layer B.Cu) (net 19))
 (segment (start 106.933 148.49) (end 108.183 149.74) (width 0.5) (layer B.Cu) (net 19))
 (segment (start 105.643 142.12) (end 105.643 136.85) (width 0.5) (layer B.Cu) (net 28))
 (segment (start 105.643 136.85) (end 113.253 129.24) (width 0.5) (layer B.Cu) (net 28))
 (segment (start 110.713 129.24) (end 110.713 129.745) (width 0.5) (layer B.Cu) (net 16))
 (segment (start 110.713 129.745) (end 104.393 136.065) (width 0.5) (layer B.Cu) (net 16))
 (segment (start 104.393 136.065) (end 104.393 148.45) (width 0.5) (layer B.Cu) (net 16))
 (segment (start 104.393 148.45) (end 103.103 149.74) (width 0.5) (layer B.Cu) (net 16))
 (segment (start 111.238 137.795) (end 106.038 132.595) (width 0.5) (layer F.Cu) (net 20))
 (segment (start 106.038 132.595) (end 106.038 132.195) (width 0.5) (layer F.Cu) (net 20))
 (segment (start 111.238 137.795) (end 112.013 138.57) (width 0.5) (layer B.Cu) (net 20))
 (segment (start 112.013 138.57) (end 112.013 148.45) (width 0.5) (layer B.Cu) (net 20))
 (segment (start 112.013 148.45) (end 110.723 149.74) (width 0.5) (layer B.Cu) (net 20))
 (segment (start 108.173 129.24) (end 106.038 131.375) (width 0.5) (layer B.Cu) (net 20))
 (segment (start 106.038 131.375) (end 106.038 132.195) (width 0.5) (layer B.Cu) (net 20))
 (via (at 111.238 137.795) (size 1.6) (drill 0.8) (layers F.Cu B.Cu) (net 20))
 (via (at 106.038 132.195) (size 1.6) (drill 0.8) (layers F.Cu B.Cu) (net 20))
 (segment (start 118.333 121.62) (end 122.123 125.41) (width 0.5) (layer B.Cu) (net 17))
 (segment (start 122.123 125.41) (end 122.123 130.23) (width 0.5) (layer B.Cu) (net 17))
 (segment (start 122.123 130.23) (end 123.423 131.53) (width 0.5) (layer B.Cu) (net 17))
 (segment (start 123.423 131.53) (end 123.423 142.12) (width 0.5) (layer B.Cu) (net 17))
 (segment (start 109.613 139.145) (end 104.438 133.97) (width 0.5) (layer F.Cu) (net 24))
 (segment (start 104.438 133.97) (end 104.438 133.57) (width 0.5) (layer F.Cu) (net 24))
 (segment (start 110.723 142.12) (end 110.723 140.255) (width 0.5) (layer B.Cu) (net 24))
 (segment (start 110.723 140.255) (end 109.613 139.145) (width 0.5) (layer B.Cu) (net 24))
 (segment (start 105.633 129.24) (end 104.438 130.435) (width 0.5) (layer B.Cu) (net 24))
 (segment (start 104.438 130.435) (end 104.438 133.57) (width 0.5) (layer B.Cu) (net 24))
 (via (at 109.613 139.145) (size 1.6) (drill 0.8) (layers F.Cu B.Cu) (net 24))
 (via (at 104.438 133.57) (size 1.6) (drill 0.8) (layers F.Cu B.Cu) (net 24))
 (segment (start 120.873 121.62) (end 122.398 123.145) (width 0.5) (layer B.Cu) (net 15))
 (segment (start 122.398 123.145) (end 124.438 123.145) (width 0.5) (layer B.Cu) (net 15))
 (segment (start 124.438 123.145) (end 125.038 122.545) (width 0.5) (layer B.Cu) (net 15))
 (segment (start 125.038 122.545) (end 125.038 121.295) (width 0.5) (layer B.Cu) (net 15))
 (segment (start 125.038 121.295) (end 126.043 120.29) (width 0.5) (layer B.Cu) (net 15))
 (segment (start 126.043 120.29) (end 126.043 118.14) (width 0.5) (layer B.Cu) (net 15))
 (segment (start 126.043 118.14) (end 126.838 117.345) (width 0.5) (layer B.Cu) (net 15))
 (segment (start 126.838 117.345) (end 128.688 117.345) (width 0.5) (layer B.Cu) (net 15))
 (segment (start 128.688 117.345) (end 129.833 118.49) (width 0.5) (layer B.Cu) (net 15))
 (segment (start 129.833 118.49) (end 129.833 118.945) (width 0.5) (layer B.Cu) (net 15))
 (segment (start 120.873 121.62) (end 120.463 121.21) (width 0.5) (layer B.Cu) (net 15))
 (segment (start 103.103 142.12) (end 103.103 129.25) (width 0.5) (layer B.Cu) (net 30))
 (segment (start 103.103 129.25) (end 103.093 129.24) (width 0.5) (layer B.Cu) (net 30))
 (segment (start 123.413 121.62) (end 123.413 120.145) (width 0.5) (layer B.Cu) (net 12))
 (segment (start 123.413 120.145) (end 122.213 118.945) (width 0.5) (layer B.Cu) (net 12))
 (segment (start 123.423 149.74) (end 121.903 148.22) (width 0.5) (layer B.Cu) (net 29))
 (segment (start 121.903 148.22) (end 120.363 148.22) (width 0.5) (layer B.Cu) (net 29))
 (segment (start 120.363 148.22) (end 119.593 148.99) (width 0.5) (layer B.Cu) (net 29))
 (segment (start 119.593 148.99) (end 119.593 152.34) (width 0.5) (layer B.Cu) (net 29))
 (segment (start 119.593 152.34) (end 116.363 155.57) (width 0.5) (layer B.Cu) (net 29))
 (segment (start 116.363 155.57) (end 114.713 155.57) (width 0.5) (layer B.Cu) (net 29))
 (segment (start 114.713 155.57) (end 113.863 156.42) (width 0.5) (layer B.Cu) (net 29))
 (segment (start 113.863 156.42) (end 113.863 158.52) (width 0.5) (layer B.Cu) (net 29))
 (segment (start 113.863 158.52) (end 114.663 159.32) (width 0.5) (layer B.Cu) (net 29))
 (segment (start 114.663 159.32) (end 115.613 159.32) (width 0.5) (layer B.Cu) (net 29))
 (segment (start 115.613 157.32) (end 120.883 152.05) (width 0.5) (layer B.Cu) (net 27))
 (segment (start 120.883 152.05) (end 120.883 149.74) (width 0.5) (layer B.Cu) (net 27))
 (segment (start 116.788 105.37) (end 119.288 107.87) (width 0.5) (layer B.Cu) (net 5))
 (segment (start 119.288 107.87) (end 122.988 107.87) (width 0.5) (layer B.Cu) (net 5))
 (segment (start 122.988 107.87) (end 125.988 104.87) (width 0.5) (layer B.Cu) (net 5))
 (segment (start 125.988 104.87) (end 128.713 104.87) (width 0.5) (layer B.Cu) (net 5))
 (segment (start 128.713 104.87) (end 129.763 105.92) (width 0.5) (layer B.Cu) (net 5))
 (segment (start 129.763 105.92) (end 129.763 108.855) (width 0.5) (layer B.Cu) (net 5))
 (segment (start 129.763 108.855) (end 127.293 111.325) (width 0.5) (layer B.Cu) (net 5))
 (segment (start 106.113 102.015) (end 113.433 102.015) (width 0.5) (layer B.Cu) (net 5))
 (segment (start 113.433 102.015) (end 116.788 105.37) (width 0.5) (layer B.Cu) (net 5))
 (segment (start 111.788 105.53) (end 111.788 105.37) (width 0.5) (layer B.Cu) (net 14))
 (segment (start 118.153 112.67) (end 111.788 106.305) (width 0.5) (layer B.Cu) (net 14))
 (segment (start 111.788 106.305) (end 111.788 105.53) (width 0.5) (layer B.Cu) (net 14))
 (segment (start 124.753 111.325) (end 124.753 112.155) (width 0.5) (layer B.Cu) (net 14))
 (segment (start 124.753 112.155) (end 123.313 113.595) (width 0.5) (layer B.Cu) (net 14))
 (segment (start 123.313 113.595) (end 119.078 113.595) (width 0.5) (layer B.Cu) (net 14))
 (segment (start 119.078 113.595) (end 118.153 112.67) (width 0.5) (layer B.Cu) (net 14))
 (segment (start 111.788 105.53) (end 111.788 105.37) (width 0.5) (layer B.Cu) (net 14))
 (segment (start 118.343 142.12) (end 120.143 143.92) (width 0.5) (layer B.Cu) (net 9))
 (segment (start 120.143 143.92) (end 123.613 143.92) (width 0.5) (layer B.Cu) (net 9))
 (segment (start 123.613 143.92) (end 124.673 142.86) (width 0.5) (layer B.Cu) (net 9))
 (segment (start 124.673 142.86) (end 124.673 142.71) (width 0.5) (layer B.Cu) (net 9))
 (segment (start 124.673 142.71) (end 124.713 142.67) (width 0.5) (layer B.Cu) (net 9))
 (segment (start 124.713 142.67) (end 124.713 139.92) (width 0.5) (layer B.Cu) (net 9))
 (segment (start 124.713 139.92) (end 127.513 137.12) (width 0.5) (layer B.Cu) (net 9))
 (segment (start 127.513 137.12) (end 127.513 135.77) (width 0.5) (layer B.Cu) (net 9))
 (segment (start 118.343 142.12) (end 118.343 140.77) (width 0.5) (layer B.Cu) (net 9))
 (segment (start 118.343 140.77) (end 120.763 138.35) (width 0.5) (layer B.Cu) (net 9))
 (segment (start 106.113 107.095) (end 107.313 108.295) (width 0.5) (layer B.Cu) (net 4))
 (segment (start 107.313 108.295) (end 109.888 108.295) (width 0.5) (layer B.Cu) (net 4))
 (segment (start 109.888 108.295) (end 114.263 112.67) (width 0.5) (layer B.Cu) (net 4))
 (segment (start 114.263 112.67) (end 115.613 112.67) (width 0.5) (layer B.Cu) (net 4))
 (segment (start 108.113 152.84) (end 108.113 152.635) (width 0.5) (layer B.Cu) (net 7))
 (segment (start 108.113 152.945) (end 108.113 152.84) (width 0.5) (layer B.Cu) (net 7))
 (segment (start 108.588 152.84) (end 108.588 152.685) (width 0.5) (layer B.Cu) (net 7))
 (segment (start 108.588 152.685) (end 105.643 149.74) (width 0.5) (layer B.Cu) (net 7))
 (segment (start 108.588 152.995) (end 108.588 152.84) (width 0.5) (layer B.Cu) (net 7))
 (segment (start 108.588 152.84) (end 108.113 152.84) (width 0.5) (layer B.Cu) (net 7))
 (segment (start 127.438 107.095) (end 126.238 108.295) (width 0.5) (layer B.Cu) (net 6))
 (segment (start 126.238 108.295) (end 125.243 108.295) (width 0.5) (layer B.Cu) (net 6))
 (segment (start 125.243 108.295) (end 122.213 111.325) (width 0.5) (layer B.Cu) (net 6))
 (segment (start 127.438 107.4) (end 127.438 107.095) (width 0.5) (layer B.Cu) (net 6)))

